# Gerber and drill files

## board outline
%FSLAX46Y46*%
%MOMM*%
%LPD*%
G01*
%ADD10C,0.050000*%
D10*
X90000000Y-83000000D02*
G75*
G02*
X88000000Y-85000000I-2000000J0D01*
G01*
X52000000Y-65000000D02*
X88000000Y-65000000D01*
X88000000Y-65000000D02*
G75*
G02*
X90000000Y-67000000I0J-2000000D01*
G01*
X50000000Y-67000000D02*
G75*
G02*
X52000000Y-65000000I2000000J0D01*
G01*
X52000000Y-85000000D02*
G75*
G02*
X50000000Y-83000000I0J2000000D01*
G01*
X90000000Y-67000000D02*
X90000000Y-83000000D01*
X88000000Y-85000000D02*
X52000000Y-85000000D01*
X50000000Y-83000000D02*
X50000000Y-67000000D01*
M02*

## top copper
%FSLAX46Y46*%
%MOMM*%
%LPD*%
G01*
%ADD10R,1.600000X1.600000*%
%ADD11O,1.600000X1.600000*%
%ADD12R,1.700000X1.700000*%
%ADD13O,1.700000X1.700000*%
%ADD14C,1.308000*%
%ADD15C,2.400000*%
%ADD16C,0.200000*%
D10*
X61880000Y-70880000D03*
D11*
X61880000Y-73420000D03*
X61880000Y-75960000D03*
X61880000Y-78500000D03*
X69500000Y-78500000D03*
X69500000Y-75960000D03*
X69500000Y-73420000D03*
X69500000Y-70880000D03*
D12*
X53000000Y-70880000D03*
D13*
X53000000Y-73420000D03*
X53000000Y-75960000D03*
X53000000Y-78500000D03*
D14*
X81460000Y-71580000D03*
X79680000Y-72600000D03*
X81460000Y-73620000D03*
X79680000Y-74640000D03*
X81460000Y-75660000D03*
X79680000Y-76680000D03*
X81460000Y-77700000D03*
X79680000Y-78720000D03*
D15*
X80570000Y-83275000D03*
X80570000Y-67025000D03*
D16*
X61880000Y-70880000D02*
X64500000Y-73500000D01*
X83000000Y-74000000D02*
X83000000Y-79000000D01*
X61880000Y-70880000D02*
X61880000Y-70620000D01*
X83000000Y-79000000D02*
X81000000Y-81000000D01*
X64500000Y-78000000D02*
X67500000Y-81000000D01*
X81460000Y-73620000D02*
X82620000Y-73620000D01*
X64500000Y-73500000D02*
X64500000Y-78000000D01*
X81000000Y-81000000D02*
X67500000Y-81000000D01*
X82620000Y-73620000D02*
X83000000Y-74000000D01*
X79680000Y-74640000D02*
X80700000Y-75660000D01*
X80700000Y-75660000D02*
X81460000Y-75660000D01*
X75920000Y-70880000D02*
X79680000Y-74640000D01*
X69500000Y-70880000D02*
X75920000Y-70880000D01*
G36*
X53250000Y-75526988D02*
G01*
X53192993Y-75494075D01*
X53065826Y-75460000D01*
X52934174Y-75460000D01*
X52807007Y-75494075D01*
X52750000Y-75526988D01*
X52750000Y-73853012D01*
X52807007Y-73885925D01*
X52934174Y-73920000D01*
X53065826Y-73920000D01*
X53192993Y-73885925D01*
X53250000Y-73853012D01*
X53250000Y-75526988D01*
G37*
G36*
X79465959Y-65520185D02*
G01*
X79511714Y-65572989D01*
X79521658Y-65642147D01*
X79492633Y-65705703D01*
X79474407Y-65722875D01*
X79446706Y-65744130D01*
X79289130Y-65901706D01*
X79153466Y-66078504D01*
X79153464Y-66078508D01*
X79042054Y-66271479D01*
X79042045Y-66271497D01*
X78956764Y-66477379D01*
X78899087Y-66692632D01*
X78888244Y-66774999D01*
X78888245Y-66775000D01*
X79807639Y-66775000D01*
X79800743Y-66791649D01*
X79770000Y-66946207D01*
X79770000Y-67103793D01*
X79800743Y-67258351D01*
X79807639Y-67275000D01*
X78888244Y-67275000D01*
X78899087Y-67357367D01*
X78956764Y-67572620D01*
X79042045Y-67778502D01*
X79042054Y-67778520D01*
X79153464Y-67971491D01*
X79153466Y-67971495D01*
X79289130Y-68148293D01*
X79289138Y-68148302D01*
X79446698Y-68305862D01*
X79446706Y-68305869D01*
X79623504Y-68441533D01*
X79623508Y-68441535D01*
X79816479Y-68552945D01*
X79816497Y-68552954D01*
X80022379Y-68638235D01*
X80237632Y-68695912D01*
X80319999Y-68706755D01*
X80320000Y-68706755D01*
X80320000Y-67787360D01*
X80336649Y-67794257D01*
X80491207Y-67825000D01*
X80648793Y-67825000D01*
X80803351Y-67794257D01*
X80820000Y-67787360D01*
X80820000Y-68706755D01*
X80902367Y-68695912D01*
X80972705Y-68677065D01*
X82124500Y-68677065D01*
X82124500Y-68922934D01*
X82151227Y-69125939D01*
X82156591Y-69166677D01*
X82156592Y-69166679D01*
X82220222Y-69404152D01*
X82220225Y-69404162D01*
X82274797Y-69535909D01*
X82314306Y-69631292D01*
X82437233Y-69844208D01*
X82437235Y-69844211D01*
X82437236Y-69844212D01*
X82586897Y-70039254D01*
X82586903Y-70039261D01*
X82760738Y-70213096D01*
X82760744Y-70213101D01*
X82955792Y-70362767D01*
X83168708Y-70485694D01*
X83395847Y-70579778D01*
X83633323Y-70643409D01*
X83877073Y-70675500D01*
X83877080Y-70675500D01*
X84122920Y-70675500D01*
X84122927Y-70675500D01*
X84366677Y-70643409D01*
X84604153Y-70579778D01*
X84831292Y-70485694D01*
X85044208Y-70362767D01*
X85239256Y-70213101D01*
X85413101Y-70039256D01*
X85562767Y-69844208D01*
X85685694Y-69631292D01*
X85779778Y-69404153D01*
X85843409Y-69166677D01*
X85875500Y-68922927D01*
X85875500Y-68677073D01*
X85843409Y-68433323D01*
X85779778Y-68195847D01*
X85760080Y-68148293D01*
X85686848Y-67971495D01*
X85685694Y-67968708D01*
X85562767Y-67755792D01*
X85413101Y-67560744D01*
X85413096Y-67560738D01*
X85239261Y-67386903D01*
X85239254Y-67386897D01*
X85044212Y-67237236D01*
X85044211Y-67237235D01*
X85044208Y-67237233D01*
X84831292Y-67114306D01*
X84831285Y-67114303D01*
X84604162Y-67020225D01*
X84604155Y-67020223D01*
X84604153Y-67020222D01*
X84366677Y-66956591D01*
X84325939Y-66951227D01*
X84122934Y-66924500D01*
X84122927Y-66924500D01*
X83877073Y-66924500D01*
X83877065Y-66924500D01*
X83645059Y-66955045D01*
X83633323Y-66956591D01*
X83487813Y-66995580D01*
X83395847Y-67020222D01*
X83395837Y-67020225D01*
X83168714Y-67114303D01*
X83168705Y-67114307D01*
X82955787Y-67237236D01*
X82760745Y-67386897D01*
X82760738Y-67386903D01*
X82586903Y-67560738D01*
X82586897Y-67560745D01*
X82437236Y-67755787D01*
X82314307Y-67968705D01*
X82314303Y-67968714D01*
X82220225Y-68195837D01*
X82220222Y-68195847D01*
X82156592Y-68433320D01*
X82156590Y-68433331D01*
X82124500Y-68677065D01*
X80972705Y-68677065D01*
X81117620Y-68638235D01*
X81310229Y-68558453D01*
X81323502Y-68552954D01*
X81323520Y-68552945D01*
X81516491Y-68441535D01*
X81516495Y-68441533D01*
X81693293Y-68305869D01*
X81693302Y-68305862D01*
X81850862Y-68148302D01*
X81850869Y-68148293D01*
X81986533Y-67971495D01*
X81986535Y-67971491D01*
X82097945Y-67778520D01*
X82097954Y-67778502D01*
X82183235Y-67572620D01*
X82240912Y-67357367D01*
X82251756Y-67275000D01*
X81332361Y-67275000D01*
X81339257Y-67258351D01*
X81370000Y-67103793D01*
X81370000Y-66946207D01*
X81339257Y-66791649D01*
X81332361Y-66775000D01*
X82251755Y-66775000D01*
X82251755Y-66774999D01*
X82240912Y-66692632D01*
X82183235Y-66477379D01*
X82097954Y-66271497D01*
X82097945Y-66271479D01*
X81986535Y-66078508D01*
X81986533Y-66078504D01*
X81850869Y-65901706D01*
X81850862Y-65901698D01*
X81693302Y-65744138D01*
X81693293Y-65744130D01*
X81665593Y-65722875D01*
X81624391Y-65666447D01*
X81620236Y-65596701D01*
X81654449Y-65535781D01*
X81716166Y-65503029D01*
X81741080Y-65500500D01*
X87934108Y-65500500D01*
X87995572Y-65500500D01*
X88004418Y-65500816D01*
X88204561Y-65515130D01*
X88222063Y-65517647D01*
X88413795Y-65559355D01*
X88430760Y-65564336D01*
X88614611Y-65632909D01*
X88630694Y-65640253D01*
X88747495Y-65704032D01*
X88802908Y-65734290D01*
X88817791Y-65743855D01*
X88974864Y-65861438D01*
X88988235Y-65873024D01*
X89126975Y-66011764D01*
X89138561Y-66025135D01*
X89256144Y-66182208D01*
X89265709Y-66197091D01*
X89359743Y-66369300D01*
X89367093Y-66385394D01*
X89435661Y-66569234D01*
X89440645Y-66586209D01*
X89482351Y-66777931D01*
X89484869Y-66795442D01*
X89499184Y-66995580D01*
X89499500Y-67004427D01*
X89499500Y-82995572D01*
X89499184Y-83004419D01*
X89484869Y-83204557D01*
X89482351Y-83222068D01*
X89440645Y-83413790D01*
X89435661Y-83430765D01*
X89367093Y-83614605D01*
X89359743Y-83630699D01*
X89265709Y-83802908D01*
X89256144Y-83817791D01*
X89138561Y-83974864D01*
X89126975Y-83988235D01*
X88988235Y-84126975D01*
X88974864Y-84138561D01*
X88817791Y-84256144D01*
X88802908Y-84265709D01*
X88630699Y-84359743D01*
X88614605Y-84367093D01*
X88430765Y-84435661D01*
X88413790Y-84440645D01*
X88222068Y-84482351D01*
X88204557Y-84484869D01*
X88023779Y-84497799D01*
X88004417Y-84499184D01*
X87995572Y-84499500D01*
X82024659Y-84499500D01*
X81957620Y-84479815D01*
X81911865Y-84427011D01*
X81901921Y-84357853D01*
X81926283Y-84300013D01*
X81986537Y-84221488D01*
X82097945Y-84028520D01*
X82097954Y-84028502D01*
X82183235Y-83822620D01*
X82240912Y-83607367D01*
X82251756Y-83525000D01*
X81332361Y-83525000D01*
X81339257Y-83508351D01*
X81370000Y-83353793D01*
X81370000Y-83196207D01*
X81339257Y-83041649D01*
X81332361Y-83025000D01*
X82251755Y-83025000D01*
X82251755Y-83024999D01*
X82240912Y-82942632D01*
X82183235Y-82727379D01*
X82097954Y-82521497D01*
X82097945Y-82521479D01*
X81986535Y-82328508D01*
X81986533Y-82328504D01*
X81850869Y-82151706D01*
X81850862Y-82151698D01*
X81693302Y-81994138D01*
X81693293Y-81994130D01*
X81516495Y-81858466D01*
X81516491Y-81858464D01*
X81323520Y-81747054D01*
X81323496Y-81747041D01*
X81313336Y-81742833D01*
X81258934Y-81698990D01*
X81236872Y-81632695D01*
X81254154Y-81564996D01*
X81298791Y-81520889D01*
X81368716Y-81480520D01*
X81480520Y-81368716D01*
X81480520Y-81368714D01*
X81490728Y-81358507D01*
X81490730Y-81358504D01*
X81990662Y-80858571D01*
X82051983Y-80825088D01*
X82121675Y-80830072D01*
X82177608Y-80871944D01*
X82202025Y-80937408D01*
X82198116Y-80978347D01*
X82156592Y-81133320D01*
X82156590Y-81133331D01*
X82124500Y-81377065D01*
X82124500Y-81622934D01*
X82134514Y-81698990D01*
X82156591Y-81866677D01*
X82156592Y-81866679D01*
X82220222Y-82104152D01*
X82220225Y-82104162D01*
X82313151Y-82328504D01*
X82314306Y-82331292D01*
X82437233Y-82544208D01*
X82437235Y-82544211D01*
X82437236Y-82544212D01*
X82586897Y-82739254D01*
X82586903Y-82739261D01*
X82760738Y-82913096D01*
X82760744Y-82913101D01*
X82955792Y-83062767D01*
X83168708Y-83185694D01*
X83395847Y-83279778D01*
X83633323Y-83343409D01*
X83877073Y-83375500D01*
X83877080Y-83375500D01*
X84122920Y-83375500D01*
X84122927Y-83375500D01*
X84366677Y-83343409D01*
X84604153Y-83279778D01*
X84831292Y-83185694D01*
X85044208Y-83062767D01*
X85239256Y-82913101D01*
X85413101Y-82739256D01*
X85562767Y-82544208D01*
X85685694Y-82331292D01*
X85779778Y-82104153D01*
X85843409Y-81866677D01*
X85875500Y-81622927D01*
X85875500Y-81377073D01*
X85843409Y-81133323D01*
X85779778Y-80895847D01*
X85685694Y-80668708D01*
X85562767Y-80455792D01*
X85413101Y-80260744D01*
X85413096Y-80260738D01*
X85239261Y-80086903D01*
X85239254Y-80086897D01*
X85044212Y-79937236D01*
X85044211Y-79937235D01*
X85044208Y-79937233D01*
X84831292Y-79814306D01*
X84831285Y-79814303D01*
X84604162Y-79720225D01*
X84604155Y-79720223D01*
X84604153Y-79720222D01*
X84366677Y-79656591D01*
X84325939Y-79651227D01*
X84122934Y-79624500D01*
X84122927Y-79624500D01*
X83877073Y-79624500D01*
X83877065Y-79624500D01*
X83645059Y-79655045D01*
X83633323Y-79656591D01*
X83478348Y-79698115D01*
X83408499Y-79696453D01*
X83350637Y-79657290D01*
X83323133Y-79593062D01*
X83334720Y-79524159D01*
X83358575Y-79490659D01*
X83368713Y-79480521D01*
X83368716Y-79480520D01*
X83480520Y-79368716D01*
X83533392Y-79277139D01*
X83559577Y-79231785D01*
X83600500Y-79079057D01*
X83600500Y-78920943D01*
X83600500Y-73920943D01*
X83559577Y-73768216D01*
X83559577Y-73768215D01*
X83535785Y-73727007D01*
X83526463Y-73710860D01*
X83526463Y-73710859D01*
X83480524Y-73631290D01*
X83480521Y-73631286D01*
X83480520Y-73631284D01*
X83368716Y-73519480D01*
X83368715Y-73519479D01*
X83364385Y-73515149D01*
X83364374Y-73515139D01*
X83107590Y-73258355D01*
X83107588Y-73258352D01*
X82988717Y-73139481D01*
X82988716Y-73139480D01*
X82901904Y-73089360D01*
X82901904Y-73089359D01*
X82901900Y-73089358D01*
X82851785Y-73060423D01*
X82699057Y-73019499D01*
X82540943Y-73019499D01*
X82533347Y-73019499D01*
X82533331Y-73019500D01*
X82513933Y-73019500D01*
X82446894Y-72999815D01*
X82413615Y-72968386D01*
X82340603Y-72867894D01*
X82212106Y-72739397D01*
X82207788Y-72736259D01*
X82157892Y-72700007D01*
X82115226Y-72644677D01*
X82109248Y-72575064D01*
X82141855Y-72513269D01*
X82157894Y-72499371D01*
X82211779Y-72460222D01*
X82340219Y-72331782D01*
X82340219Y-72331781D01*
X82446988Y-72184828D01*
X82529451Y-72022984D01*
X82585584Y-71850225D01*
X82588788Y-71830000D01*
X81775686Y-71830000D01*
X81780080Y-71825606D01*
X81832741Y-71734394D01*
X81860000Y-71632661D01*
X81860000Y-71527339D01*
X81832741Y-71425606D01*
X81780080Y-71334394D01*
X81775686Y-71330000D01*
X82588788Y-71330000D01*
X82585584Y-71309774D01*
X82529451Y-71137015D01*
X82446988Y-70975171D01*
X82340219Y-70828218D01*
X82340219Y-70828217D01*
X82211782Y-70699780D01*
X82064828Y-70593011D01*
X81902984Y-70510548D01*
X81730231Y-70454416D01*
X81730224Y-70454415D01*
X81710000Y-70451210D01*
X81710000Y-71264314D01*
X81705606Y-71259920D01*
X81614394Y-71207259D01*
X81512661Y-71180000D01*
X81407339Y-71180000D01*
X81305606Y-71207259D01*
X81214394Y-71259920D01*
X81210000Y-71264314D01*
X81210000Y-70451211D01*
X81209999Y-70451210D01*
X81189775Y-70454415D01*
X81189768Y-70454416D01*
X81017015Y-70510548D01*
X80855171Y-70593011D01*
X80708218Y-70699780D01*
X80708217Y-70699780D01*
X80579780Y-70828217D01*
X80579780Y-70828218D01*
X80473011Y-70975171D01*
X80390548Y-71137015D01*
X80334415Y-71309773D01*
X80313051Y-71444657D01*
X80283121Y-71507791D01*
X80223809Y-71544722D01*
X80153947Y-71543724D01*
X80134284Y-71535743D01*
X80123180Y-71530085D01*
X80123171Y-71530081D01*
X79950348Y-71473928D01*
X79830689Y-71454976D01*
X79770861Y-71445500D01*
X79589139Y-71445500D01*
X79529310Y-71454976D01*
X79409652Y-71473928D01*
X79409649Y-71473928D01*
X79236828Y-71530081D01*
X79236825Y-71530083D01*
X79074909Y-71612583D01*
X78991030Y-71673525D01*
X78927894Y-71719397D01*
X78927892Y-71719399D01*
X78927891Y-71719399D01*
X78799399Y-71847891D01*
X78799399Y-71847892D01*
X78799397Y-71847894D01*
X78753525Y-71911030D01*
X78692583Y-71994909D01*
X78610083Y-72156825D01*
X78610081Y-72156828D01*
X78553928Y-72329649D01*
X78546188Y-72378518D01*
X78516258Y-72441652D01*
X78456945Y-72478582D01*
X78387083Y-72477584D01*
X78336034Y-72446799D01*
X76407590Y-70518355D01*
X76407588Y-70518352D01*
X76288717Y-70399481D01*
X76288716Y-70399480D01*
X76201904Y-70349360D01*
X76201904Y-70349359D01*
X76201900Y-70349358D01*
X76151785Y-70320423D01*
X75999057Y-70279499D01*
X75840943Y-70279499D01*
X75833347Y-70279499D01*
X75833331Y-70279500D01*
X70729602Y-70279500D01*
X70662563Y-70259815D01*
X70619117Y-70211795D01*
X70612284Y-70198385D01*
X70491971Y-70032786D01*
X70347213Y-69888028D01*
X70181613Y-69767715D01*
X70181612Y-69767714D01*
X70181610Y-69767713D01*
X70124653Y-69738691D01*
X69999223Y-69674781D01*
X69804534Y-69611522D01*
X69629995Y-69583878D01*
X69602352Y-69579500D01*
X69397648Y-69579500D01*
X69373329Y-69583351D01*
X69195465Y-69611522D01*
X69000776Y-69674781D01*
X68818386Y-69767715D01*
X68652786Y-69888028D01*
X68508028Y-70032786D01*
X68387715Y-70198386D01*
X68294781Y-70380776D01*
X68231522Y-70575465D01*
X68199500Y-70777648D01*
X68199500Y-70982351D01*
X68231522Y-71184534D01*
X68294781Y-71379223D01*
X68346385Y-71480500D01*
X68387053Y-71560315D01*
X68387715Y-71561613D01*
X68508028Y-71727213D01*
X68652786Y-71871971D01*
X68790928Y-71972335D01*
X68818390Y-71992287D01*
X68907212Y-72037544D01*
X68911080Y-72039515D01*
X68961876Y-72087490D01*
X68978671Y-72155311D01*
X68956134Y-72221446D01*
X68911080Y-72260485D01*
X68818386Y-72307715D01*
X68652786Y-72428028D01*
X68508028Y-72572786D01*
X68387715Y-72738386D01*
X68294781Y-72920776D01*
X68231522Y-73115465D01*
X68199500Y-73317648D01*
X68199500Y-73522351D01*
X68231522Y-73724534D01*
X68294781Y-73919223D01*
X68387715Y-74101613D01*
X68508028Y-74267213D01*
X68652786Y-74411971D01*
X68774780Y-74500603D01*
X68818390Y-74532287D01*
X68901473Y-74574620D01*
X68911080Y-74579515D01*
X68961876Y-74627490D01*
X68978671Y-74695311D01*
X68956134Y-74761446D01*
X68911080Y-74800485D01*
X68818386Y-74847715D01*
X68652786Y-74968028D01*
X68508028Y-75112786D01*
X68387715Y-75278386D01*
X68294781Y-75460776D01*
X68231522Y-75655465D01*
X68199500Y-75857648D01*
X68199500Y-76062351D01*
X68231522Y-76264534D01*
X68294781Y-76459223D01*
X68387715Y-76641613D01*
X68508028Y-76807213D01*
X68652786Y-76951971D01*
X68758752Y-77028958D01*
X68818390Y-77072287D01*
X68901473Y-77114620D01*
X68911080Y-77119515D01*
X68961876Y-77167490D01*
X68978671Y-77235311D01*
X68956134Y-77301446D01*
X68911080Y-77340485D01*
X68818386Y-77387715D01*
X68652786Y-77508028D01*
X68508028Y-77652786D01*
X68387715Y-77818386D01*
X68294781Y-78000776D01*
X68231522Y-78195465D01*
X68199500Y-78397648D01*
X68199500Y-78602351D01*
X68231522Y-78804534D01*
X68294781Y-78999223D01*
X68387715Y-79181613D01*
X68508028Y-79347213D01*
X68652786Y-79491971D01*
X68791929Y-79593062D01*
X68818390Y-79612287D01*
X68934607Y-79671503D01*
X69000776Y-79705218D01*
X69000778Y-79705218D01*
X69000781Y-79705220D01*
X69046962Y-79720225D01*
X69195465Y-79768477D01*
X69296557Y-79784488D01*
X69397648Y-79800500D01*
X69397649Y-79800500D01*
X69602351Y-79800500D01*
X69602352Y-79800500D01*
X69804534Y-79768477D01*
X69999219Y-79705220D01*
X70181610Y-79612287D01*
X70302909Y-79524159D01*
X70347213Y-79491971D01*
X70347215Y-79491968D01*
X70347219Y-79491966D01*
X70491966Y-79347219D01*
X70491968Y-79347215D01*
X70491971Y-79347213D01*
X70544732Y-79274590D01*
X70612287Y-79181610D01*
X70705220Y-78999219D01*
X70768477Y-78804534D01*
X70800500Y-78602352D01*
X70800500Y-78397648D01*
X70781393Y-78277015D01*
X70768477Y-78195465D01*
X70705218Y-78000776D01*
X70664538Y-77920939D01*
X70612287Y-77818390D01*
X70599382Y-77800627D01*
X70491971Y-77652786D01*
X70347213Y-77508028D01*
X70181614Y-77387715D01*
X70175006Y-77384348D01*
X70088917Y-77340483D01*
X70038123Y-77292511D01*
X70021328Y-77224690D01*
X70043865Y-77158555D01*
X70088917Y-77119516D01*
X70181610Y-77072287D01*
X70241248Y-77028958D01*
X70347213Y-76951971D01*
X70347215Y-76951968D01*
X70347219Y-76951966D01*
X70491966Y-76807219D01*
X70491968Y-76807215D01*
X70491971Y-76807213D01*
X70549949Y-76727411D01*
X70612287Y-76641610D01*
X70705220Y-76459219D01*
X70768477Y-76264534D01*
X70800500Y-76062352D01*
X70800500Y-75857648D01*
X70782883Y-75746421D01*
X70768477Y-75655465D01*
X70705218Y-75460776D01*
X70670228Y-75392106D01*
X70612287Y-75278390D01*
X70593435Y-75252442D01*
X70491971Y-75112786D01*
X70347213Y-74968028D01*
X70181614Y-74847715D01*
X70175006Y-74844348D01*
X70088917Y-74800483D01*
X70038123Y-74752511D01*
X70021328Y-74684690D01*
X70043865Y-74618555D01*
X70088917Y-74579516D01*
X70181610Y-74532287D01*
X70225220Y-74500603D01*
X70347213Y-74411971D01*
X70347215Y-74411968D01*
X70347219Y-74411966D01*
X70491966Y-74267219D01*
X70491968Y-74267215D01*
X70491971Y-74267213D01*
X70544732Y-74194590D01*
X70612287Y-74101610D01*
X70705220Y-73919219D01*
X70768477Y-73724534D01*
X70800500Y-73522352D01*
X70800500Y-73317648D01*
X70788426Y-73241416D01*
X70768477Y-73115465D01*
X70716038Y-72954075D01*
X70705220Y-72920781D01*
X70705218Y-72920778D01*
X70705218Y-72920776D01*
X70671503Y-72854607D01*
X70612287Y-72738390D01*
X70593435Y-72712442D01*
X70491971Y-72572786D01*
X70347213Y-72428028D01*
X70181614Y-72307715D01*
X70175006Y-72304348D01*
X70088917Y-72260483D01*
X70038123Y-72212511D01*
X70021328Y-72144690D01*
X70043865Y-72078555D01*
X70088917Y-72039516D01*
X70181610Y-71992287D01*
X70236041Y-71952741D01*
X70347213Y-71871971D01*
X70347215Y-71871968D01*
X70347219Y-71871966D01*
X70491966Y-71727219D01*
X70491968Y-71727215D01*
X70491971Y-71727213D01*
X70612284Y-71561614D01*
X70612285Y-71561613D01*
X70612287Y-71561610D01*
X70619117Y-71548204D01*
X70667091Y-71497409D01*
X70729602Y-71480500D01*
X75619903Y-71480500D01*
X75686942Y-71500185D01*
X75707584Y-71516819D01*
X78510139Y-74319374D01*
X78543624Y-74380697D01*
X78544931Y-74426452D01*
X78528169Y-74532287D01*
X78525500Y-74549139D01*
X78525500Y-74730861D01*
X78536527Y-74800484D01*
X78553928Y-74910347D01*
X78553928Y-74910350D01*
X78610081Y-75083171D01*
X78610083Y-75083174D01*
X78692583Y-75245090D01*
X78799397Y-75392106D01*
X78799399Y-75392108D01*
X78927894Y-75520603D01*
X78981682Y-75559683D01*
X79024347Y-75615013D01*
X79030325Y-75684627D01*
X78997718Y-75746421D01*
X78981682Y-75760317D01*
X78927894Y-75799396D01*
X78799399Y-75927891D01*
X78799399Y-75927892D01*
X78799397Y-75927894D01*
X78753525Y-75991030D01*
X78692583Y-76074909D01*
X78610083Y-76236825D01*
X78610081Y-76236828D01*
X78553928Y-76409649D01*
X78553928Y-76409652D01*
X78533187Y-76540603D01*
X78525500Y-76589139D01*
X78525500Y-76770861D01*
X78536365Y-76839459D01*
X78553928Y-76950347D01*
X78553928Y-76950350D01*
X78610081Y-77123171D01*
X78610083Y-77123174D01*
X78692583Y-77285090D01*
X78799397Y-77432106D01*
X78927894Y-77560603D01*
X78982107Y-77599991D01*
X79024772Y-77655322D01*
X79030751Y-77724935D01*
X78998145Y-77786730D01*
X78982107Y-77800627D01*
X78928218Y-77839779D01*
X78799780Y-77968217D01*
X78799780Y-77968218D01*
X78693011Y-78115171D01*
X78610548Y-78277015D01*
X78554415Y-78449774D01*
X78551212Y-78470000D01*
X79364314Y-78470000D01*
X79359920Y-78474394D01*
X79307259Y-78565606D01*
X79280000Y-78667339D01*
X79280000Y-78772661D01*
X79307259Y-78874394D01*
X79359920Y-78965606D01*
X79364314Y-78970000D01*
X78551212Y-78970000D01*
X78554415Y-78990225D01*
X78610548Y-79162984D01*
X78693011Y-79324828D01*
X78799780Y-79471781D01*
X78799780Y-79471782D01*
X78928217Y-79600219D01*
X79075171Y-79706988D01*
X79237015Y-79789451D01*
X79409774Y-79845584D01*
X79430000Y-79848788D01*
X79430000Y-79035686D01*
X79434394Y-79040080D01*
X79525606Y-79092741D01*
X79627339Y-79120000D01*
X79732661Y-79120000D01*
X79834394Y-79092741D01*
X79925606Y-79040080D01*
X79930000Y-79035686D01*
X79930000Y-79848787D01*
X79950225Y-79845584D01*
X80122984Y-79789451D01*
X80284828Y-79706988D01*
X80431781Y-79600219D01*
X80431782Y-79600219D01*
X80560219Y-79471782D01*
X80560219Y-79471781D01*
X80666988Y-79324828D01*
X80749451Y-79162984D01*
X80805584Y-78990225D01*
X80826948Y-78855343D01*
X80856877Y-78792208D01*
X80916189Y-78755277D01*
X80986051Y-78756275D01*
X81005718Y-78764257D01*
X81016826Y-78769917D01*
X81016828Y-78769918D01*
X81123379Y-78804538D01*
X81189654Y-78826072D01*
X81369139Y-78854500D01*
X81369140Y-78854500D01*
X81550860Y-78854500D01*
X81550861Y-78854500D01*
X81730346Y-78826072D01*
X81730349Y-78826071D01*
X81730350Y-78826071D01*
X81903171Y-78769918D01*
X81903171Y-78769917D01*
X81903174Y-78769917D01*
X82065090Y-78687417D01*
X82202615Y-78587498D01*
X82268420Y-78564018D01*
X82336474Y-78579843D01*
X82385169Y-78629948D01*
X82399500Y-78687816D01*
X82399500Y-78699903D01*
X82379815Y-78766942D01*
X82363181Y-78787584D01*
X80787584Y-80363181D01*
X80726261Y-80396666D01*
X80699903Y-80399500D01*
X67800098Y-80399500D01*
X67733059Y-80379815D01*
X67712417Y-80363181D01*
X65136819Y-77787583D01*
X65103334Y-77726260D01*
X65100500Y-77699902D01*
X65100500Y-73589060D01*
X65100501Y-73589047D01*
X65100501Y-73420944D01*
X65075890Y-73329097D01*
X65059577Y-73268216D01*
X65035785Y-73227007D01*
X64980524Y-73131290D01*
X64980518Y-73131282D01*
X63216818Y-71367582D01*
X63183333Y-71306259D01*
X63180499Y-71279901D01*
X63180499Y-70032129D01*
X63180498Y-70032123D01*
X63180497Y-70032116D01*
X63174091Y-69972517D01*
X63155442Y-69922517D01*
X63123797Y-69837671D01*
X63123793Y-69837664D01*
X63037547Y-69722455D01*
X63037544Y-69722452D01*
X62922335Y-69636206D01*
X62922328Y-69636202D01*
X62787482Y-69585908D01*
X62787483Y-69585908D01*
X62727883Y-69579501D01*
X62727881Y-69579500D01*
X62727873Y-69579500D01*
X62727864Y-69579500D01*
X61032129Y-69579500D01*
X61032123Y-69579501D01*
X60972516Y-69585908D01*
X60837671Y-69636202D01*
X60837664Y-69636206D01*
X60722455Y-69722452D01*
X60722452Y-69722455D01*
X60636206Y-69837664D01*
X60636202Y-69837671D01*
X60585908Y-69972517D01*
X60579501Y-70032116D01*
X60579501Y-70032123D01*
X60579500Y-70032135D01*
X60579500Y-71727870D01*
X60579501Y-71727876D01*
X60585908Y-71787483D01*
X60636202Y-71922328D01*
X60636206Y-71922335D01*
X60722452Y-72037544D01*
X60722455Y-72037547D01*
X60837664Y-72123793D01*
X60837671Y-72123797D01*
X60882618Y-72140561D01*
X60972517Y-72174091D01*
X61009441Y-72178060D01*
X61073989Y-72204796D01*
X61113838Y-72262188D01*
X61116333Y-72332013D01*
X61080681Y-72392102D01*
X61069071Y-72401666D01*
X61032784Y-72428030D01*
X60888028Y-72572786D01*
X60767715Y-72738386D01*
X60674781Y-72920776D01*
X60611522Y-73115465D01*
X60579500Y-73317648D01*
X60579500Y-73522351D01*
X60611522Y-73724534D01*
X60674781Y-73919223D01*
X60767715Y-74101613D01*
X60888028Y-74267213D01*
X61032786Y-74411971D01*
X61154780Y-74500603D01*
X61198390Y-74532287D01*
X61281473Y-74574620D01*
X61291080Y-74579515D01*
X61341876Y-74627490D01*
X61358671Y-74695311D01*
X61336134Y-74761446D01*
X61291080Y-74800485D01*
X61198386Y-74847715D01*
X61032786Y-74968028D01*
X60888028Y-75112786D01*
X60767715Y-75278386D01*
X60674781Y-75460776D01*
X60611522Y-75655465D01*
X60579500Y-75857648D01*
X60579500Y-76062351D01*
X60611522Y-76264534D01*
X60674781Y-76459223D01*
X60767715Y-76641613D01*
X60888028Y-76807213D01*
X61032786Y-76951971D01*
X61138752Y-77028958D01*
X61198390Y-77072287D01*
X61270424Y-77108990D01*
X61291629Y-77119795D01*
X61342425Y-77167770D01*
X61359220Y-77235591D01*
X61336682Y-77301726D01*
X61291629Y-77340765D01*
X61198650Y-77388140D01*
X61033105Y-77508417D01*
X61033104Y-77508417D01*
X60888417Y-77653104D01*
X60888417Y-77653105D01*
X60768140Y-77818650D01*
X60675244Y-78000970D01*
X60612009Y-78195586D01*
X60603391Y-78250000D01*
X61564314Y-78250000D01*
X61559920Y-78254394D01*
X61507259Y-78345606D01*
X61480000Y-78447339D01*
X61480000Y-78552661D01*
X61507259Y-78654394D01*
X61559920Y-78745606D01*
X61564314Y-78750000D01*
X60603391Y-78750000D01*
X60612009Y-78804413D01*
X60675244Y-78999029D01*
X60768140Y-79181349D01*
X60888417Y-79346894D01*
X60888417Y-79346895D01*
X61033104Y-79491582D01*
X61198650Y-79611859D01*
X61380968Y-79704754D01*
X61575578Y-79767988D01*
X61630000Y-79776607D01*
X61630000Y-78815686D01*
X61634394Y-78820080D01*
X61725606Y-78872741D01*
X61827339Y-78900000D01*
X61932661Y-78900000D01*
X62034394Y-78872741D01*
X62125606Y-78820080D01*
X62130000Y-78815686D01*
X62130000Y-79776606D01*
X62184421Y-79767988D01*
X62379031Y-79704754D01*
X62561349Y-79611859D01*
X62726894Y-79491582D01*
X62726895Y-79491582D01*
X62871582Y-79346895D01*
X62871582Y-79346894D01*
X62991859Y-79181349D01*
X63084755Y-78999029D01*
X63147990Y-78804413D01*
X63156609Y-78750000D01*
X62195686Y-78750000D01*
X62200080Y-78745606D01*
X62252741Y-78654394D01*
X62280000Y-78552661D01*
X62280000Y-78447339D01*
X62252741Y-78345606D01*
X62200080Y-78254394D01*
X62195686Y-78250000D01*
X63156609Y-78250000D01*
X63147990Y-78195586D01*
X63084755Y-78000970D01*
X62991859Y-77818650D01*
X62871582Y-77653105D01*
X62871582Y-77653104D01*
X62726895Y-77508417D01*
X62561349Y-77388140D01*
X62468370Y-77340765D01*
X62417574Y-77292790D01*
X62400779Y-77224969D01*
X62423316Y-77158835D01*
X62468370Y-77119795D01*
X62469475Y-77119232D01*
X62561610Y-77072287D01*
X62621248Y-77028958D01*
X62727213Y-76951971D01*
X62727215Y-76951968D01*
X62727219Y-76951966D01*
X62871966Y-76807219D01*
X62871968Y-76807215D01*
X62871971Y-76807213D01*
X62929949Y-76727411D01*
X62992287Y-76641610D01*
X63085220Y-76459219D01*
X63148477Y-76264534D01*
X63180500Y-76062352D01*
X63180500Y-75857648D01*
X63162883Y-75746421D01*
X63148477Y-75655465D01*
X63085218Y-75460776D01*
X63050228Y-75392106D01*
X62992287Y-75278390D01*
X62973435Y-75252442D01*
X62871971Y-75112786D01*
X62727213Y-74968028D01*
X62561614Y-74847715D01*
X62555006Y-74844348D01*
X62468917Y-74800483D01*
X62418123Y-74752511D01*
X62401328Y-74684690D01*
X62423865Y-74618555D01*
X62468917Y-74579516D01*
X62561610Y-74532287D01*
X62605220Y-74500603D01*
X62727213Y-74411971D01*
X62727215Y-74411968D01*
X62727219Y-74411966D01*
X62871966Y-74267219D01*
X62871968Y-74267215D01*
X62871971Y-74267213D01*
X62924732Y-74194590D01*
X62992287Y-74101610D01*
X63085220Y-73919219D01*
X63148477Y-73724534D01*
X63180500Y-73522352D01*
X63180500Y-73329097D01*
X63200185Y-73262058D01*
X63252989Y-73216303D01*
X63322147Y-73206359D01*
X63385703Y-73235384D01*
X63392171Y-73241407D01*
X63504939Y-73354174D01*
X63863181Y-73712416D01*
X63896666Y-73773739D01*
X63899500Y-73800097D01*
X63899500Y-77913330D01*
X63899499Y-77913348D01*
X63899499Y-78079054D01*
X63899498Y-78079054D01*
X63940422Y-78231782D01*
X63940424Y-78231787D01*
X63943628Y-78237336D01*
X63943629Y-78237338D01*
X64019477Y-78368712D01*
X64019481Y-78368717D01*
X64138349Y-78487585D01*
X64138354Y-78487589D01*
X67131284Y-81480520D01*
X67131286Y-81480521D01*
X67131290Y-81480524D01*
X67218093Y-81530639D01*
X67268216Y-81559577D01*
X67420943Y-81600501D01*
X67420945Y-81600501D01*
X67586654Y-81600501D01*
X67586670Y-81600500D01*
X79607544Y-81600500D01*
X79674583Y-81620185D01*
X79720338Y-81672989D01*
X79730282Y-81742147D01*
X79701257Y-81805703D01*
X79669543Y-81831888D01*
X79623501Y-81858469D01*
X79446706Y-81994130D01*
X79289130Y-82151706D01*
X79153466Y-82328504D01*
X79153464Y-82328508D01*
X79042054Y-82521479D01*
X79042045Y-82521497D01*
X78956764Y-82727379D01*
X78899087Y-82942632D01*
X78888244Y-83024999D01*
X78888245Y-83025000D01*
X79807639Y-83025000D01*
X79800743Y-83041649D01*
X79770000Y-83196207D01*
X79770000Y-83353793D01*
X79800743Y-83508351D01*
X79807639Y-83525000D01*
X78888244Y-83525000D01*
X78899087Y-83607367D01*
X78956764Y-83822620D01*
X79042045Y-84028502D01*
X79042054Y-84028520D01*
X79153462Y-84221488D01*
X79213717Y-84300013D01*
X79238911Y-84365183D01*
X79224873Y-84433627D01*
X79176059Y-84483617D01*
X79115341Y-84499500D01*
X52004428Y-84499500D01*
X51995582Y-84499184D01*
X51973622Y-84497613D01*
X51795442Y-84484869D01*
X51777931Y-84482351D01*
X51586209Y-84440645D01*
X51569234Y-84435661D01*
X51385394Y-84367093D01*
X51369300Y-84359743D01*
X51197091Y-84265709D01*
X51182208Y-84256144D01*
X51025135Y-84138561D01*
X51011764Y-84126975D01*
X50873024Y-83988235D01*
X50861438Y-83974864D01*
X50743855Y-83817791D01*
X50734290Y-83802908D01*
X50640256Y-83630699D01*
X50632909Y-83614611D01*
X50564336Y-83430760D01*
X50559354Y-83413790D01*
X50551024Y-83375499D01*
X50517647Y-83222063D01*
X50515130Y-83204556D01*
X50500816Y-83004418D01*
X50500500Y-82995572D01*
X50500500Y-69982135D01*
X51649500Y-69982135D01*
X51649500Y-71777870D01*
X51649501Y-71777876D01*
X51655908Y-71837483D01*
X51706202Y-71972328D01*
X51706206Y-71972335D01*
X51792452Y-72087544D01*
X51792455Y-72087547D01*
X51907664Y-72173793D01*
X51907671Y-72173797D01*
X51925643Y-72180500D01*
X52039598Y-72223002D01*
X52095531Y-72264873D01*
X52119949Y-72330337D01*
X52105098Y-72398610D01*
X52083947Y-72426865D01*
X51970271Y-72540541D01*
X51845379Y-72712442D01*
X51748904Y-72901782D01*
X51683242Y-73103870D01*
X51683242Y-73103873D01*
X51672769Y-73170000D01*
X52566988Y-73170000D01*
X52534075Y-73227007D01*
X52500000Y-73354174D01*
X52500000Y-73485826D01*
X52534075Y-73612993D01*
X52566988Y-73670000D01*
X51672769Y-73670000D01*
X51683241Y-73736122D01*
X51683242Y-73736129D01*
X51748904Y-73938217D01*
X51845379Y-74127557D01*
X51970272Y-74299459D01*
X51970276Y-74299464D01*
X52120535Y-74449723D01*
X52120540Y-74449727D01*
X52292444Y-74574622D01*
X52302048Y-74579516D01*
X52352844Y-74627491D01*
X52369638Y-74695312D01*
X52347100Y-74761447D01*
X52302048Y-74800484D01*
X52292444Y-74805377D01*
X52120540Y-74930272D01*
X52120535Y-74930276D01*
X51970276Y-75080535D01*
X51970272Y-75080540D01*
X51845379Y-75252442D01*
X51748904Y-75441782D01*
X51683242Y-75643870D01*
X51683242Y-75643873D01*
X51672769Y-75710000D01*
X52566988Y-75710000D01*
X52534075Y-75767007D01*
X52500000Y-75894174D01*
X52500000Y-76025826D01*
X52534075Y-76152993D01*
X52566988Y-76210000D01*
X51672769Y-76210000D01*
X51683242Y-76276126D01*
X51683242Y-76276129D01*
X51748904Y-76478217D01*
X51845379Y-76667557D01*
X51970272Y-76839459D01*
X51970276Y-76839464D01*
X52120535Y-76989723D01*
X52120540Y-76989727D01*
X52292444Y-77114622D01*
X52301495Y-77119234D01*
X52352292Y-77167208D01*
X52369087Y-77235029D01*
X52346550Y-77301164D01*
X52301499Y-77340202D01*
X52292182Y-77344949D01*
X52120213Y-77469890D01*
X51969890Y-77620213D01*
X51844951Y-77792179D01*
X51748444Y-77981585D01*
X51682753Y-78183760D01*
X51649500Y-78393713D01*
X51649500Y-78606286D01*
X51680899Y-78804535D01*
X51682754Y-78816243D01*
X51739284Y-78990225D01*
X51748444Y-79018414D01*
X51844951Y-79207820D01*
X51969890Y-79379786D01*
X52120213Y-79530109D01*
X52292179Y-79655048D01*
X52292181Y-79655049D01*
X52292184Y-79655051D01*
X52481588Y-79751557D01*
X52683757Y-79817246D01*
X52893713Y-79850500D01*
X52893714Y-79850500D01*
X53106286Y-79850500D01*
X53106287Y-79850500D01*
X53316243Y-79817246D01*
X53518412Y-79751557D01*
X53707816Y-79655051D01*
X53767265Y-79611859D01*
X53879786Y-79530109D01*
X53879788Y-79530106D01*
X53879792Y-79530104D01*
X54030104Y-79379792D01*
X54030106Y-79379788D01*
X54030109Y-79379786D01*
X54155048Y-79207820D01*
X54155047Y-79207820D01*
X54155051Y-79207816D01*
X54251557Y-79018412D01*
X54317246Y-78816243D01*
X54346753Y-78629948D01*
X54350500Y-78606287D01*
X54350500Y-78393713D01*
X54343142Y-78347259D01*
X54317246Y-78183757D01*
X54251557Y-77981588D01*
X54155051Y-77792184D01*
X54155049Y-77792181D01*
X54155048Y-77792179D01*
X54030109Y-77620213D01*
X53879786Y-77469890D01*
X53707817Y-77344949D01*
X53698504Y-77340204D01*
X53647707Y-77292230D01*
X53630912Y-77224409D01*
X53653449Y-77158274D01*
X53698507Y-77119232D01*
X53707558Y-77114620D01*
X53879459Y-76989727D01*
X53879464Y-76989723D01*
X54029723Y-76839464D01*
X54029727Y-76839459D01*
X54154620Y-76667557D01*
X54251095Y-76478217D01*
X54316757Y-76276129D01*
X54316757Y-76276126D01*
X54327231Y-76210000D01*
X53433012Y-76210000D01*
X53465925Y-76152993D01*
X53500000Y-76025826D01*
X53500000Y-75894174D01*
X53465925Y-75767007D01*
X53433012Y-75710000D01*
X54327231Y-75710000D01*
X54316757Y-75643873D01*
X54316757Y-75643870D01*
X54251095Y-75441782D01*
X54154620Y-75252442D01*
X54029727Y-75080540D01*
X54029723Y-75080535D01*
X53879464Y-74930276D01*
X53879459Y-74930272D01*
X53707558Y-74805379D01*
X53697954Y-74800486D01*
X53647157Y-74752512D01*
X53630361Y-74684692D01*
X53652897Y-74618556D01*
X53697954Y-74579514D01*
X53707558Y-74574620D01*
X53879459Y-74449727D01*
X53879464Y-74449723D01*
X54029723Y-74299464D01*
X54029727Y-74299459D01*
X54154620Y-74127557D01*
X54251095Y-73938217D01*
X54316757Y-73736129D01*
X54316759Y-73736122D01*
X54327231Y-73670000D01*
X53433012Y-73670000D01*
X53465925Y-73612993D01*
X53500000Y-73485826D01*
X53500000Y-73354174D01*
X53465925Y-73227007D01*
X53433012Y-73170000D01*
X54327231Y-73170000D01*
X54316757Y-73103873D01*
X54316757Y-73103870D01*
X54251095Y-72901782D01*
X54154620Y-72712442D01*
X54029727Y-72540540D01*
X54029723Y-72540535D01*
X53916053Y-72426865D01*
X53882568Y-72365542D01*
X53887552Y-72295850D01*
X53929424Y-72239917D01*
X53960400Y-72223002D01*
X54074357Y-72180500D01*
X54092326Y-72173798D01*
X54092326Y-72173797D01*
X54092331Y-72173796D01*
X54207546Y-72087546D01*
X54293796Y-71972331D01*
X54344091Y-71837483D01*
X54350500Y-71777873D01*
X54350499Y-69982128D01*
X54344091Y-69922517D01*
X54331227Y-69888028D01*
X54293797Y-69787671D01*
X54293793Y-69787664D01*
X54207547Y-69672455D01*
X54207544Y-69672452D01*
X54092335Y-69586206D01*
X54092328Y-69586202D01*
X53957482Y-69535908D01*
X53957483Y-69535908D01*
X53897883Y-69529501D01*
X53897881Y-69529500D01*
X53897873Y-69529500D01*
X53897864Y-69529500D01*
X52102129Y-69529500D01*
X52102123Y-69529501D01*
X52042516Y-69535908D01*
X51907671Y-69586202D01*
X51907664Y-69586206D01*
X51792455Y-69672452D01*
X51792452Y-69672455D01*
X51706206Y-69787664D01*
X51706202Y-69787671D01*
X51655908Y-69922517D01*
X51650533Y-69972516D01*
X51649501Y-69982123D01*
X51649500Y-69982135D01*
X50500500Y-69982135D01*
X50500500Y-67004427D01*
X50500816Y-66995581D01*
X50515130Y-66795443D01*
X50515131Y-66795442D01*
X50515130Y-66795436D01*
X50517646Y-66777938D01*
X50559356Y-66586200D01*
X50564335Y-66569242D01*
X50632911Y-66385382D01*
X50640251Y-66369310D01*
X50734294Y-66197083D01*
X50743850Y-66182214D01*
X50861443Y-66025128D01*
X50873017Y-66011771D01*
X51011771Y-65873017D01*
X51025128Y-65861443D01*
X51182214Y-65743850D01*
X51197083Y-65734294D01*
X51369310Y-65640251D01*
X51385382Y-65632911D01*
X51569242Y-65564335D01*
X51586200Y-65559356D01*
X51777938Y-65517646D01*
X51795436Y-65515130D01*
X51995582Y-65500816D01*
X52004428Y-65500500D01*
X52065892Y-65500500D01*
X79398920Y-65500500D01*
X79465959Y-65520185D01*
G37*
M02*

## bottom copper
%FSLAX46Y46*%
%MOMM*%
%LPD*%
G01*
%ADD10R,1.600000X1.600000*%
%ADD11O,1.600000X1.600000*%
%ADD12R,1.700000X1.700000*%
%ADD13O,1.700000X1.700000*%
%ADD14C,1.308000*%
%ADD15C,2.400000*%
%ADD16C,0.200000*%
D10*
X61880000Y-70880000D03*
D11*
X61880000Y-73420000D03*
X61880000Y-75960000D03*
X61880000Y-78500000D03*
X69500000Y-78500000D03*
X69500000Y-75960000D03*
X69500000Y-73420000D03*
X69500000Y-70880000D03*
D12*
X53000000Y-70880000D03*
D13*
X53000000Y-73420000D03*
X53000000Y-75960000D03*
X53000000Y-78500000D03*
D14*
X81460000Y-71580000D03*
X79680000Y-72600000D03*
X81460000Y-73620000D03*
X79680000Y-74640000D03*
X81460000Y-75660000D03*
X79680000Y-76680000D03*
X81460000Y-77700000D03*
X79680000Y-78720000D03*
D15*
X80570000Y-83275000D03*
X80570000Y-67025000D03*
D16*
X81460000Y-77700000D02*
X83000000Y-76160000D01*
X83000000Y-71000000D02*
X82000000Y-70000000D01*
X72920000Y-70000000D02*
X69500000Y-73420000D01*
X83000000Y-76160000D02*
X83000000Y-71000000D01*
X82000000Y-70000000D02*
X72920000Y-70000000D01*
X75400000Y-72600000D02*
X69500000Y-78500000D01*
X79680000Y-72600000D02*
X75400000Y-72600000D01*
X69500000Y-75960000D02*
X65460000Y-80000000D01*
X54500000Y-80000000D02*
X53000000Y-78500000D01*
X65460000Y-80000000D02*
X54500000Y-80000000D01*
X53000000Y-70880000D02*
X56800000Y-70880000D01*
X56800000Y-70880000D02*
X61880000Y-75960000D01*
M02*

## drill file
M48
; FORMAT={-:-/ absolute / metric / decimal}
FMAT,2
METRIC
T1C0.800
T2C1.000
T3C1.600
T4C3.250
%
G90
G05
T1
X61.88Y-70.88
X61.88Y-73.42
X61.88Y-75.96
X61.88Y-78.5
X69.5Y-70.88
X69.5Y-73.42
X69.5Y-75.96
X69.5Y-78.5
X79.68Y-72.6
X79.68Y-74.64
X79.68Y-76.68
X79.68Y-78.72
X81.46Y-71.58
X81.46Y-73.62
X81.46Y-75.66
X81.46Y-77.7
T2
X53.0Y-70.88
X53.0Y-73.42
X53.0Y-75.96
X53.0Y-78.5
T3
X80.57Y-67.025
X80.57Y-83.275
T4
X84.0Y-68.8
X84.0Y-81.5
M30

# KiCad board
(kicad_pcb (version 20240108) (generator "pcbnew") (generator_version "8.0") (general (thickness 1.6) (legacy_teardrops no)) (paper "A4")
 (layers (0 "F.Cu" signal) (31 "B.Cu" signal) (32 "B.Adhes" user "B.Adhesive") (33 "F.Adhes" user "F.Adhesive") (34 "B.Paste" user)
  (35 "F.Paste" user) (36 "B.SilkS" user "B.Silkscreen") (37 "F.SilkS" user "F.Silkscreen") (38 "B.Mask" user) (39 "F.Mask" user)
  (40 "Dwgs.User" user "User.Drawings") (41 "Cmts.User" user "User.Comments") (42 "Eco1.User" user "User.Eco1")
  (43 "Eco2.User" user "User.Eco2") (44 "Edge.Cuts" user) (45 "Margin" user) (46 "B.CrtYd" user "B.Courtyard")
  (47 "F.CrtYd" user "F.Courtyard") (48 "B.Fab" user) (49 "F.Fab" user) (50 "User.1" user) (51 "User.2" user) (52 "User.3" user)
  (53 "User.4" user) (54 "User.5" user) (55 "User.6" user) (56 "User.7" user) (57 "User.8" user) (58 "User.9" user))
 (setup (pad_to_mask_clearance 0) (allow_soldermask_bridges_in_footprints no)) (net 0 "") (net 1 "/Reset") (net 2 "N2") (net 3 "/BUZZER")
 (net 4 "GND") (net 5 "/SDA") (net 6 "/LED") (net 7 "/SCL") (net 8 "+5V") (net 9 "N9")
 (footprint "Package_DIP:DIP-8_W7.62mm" (layer "F.Cu") (at 61.88 70.88)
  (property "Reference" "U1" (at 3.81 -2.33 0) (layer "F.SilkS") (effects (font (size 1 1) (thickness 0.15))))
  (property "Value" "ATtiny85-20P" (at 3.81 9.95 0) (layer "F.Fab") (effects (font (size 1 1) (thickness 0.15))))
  (pad "1" thru_hole rect (at 0 0) (size 1.6 1.6) (drill 0.8) (layers "*.Cu" "*.Mask") (remove_unused_layers no) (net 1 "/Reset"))
  (pad "2" thru_hole oval (at 0 2.54) (size 1.6 1.6) (drill 0.8) (layers "*.Cu" "*.Mask") (remove_unused_layers no) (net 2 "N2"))
  (pad "3" thru_hole oval (at 0 5.08) (size 1.6 1.6) (drill 0.8) (layers "*.Cu" "*.Mask") (remove_unused_layers no) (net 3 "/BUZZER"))
  (pad "4" thru_hole oval (at 0 7.62) (size 1.6 1.6) (drill 0.8) (layers "*.Cu" "*.Mask") (remove_unused_layers no) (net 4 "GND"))
  (pad "5" thru_hole oval (at 7.62 7.62) (size 1.6 1.6) (drill 0.8) (layers "*.Cu" "*.Mask") (remove_unused_layers no) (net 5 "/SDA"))
  (pad "6" thru_hole oval (at 7.62 5.08) (size 1.6 1.6) (drill 0.8) (layers "*.Cu" "*.Mask") (remove_unused_layers no) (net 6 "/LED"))
  (pad "7" thru_hole oval (at 7.62 2.54) (size 1.6 1.6) (drill 0.8) (layers "*.Cu" "*.Mask") (remove_unused_layers no) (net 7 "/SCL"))
  (pad "8" thru_hole oval (at 7.62 0) (size 1.6 1.6) (drill 0.8) (layers "*.Cu" "*.Mask") (remove_unused_layers no) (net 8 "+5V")))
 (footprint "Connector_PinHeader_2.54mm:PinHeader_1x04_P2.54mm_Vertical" (layer "F.Cu") (at 53 70.88)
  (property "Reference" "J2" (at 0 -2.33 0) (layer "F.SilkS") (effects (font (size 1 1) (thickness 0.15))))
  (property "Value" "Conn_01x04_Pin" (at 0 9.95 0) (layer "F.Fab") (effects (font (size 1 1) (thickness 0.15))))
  (pad "1" thru_hole rect (at 0 0) (size 1.7 1.7) (drill 1) (layers "*.Cu" "*.Mask") (remove_unused_layers no) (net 3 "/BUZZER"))
  (pad "2" thru_hole oval (at 0 2.54) (size 1.7 1.7) (drill 1) (layers "*.Cu" "*.Mask") (remove_unused_layers no) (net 4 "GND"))
  (pad "3" thru_hole oval (at 0 5.08) (size 1.7 1.7) (drill 1) (layers "*.Cu" "*.Mask") (remove_unused_layers no) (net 4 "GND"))
  (pad "4" thru_hole oval (at 0 7.62) (size 1.7 1.7) (drill 1) (layers "*.Cu" "*.Mask") (remove_unused_layers no) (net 6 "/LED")))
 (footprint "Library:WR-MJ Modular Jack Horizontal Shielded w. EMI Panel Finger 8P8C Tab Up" (layer "F.Cu") (at 81.585 75.15 90)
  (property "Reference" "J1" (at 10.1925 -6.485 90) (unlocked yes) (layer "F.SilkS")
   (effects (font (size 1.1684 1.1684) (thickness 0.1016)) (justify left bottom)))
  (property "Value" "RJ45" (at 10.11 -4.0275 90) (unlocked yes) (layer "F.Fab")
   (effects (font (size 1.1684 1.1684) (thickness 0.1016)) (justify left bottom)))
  (pad "" np_thru_hole circle (at -6.35 2.415 90) (size 3.25 3.25) (drill 3.25) (layers "*.Cu" "*.Mask"))
  (pad "" np_thru_hole circle (at 6.35 2.415 90) (size 3.25 3.25) (drill 3.25) (layers "*.Cu" "*.Mask"))
  (pad "1" thru_hole circle (at 3.57 -0.125 90) (size 1.308 1.308) (drill 0.8) (layers "*.Cu" "*.Mask") (remove_unused_layers no)
   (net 4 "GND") (solder_mask_margin 0.1016) (thermal_bridge_angle 0))
  (pad "2" thru_hole circle (at 2.55 -1.905 90) (size 1.308 1.308) (drill 0.8) (layers "*.Cu" "*.Mask") (remove_unused_layers no)
   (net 5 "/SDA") (solder_mask_margin 0.1016) (thermal_bridge_angle 0))
  (pad "3" thru_hole circle (at 1.53 -0.125 90) (size 1.308 1.308) (drill 0.8) (layers "*.Cu" "*.Mask") (remove_unused_layers no)
   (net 1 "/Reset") (solder_mask_margin 0.1016) (thermal_bridge_angle 0))
  (pad "4" thru_hole circle (at 0.51 -1.905 90) (size 1.308 1.308) (drill 0.8) (layers "*.Cu" "*.Mask") (remove_unused_layers no)
   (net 8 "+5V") (solder_mask_margin 0.1016) (thermal_bridge_angle 0))
  (pad "5" thru_hole circle (at -0.51 -0.125 90) (size 1.308 1.308) (drill 0.8) (layers "*.Cu" "*.Mask") (remove_unused_layers no)
   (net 8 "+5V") (solder_mask_margin 0.1016) (thermal_bridge_angle 0))
  (pad "6" thru_hole circle (at -1.53 -1.905 90) (size 1.308 1.308) (drill 0.8) (layers "*.Cu" "*.Mask") (remove_unused_layers no)
   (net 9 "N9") (solder_mask_margin 0.1016) (thermal_bridge_angle 0))
  (pad "7" thru_hole circle (at -2.55 -0.125 90) (size 1.308 1.308) (drill 0.8) (layers "*.Cu" "*.Mask") (remove_unused_layers no)
   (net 7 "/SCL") (solder_mask_margin 0.1016) (thermal_bridge_angle 0))
  (pad "8" thru_hole circle (at -3.57 -1.905 90) (size 1.308 1.308) (drill 0.8) (layers "*.Cu" "*.Mask") (remove_unused_layers no)
   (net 4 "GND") (solder_mask_margin 0.1016) (thermal_bridge_angle 0))
  (pad "S1" thru_hole circle (at -8.125 -1.015 90) (size 2.4 2.4) (drill 1.6) (layers "*.Cu" "*.Mask") (remove_unused_layers no)
   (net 4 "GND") (solder_mask_margin 0.1016) (thermal_bridge_angle 0))
  (pad "S2" thru_hole circle (at 8.125 -1.015 90) (size 2.4 2.4) (drill 1.6) (layers "*.Cu" "*.Mask") (remove_unused_layers no)
   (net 4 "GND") (solder_mask_margin 0.1016) (thermal_bridge_angle 0)))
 (gr_arc (start 90 83) (mid 89.414214 84.414214) (end 88 85) (locked yes) (stroke (width 0.05) (type default)) (layer "Edge.Cuts"))
 (gr_line (start 52 65) (end 88 65) (locked yes) (stroke (width 0.05) (type default)) (layer "Edge.Cuts"))
 (gr_arc (start 88 65) (mid 89.414214 65.585786) (end 90 67) (locked yes) (stroke (width 0.05) (type default)) (layer "Edge.Cuts"))
 (gr_arc (start 50 67) (mid 50.585786 65.585786) (end 52 65) (locked yes) (stroke (width 0.05) (type default)) (layer "Edge.Cuts"))
 (gr_arc (start 52 85) (mid 50.585786 84.414214) (end 50 83) (locked yes) (stroke (width 0.05) (type default)) (layer "Edge.Cuts"))
 (gr_line (start 90 67) (end 90 83) (locked yes) (stroke (width 0.05) (type default)) (layer "Edge.Cuts"))
 (gr_line (start 88 85) (end 52 85) (locked yes) (stroke (width 0.05) (type default)) (layer "Edge.Cuts"))
 (gr_line (start 50 83) (end 50 67) (locked yes) (stroke (width 0.05) (type default)) (layer "Edge.Cuts"))
 (segment (start 61.88 70.88) (end 64.5 73.5) (width 0.2) (layer "F.Cu") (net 1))
 (segment (start 83 74) (end 83 79) (width 0.2) (layer "F.Cu") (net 1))
 (segment (start 61.88 70.88) (end 61.88 70.62) (width 0.2) (layer "F.Cu") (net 1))
 (segment (start 83 79) (end 81 81) (width 0.2) (layer "F.Cu") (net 1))
 (segment (start 64.5 78) (end 67.5 81) (width 0.2) (layer "F.Cu") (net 1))
 (segment (start 81.46 73.62) (end 82.62 73.62) (width 0.2) (layer "F.Cu") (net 1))
 (segment (start 64.5 73.5) (end 64.5 78) (width 0.2) (layer "F.Cu") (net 1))
 (segment (start 81 81) (end 67.5 81) (width 0.2) (layer "F.Cu") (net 1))
 (segment (start 82.62 73.62) (end 83 74) (width 0.2) (layer "F.Cu") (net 1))
 (segment (start 81.46 77.7) (end 83 76.16) (width 0.2) (layer "B.Cu") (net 7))
 (segment (start 83 71) (end 82 70) (width 0.2) (layer "B.Cu") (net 7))
 (segment (start 72.92 70) (end 69.5 73.42) (width 0.2) (layer "B.Cu") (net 7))
 (segment (start 83 76.16) (end 83 71) (width 0.2) (layer "B.Cu") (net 7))
 (segment (start 82 70) (end 72.92 70) (width 0.2) (layer "B.Cu") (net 7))
 (segment (start 79.68 74.64) (end 80.7 75.66) (width 0.2) (layer "F.Cu") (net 8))
 (segment (start 80.7 75.66) (end 81.46 75.66) (width 0.2) (layer "F.Cu") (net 8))
 (segment (start 75.92 70.88) (end 79.68 74.64) (width 0.2) (layer "F.Cu") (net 8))
 (segment (start 69.5 70.88) (end 75.92 70.88) (width 0.2) (layer "F.Cu") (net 8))
 (segment (start 75.4 72.6) (end 69.5 78.5) (width 0.2) (layer "B.Cu") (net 5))
 (segment (start 79.68 72.6) (end 75.4 72.6) (width 0.2) (layer "B.Cu") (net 5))
 (segment (start 69.5 75.96) (end 65.46 80) (width 0.2) (layer "B.Cu") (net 6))
 (segment (start 54.5 80) (end 53 78.5) (width 0.2) (layer "B.Cu") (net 6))
 (segment (start 65.46 80) (end 54.5 80) (width 0.2) (layer "B.Cu") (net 6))
 (segment (start 53 70.88) (end 56.8 70.88) (width 0.2) (layer "B.Cu") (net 3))
 (segment (start 56.8 70.88) (end 61.88 75.96) (width 0.2) (layer "B.Cu") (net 3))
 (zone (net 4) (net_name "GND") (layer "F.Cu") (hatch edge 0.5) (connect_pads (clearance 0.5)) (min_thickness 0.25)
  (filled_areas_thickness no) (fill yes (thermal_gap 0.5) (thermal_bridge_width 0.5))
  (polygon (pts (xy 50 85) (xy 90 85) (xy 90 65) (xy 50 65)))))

